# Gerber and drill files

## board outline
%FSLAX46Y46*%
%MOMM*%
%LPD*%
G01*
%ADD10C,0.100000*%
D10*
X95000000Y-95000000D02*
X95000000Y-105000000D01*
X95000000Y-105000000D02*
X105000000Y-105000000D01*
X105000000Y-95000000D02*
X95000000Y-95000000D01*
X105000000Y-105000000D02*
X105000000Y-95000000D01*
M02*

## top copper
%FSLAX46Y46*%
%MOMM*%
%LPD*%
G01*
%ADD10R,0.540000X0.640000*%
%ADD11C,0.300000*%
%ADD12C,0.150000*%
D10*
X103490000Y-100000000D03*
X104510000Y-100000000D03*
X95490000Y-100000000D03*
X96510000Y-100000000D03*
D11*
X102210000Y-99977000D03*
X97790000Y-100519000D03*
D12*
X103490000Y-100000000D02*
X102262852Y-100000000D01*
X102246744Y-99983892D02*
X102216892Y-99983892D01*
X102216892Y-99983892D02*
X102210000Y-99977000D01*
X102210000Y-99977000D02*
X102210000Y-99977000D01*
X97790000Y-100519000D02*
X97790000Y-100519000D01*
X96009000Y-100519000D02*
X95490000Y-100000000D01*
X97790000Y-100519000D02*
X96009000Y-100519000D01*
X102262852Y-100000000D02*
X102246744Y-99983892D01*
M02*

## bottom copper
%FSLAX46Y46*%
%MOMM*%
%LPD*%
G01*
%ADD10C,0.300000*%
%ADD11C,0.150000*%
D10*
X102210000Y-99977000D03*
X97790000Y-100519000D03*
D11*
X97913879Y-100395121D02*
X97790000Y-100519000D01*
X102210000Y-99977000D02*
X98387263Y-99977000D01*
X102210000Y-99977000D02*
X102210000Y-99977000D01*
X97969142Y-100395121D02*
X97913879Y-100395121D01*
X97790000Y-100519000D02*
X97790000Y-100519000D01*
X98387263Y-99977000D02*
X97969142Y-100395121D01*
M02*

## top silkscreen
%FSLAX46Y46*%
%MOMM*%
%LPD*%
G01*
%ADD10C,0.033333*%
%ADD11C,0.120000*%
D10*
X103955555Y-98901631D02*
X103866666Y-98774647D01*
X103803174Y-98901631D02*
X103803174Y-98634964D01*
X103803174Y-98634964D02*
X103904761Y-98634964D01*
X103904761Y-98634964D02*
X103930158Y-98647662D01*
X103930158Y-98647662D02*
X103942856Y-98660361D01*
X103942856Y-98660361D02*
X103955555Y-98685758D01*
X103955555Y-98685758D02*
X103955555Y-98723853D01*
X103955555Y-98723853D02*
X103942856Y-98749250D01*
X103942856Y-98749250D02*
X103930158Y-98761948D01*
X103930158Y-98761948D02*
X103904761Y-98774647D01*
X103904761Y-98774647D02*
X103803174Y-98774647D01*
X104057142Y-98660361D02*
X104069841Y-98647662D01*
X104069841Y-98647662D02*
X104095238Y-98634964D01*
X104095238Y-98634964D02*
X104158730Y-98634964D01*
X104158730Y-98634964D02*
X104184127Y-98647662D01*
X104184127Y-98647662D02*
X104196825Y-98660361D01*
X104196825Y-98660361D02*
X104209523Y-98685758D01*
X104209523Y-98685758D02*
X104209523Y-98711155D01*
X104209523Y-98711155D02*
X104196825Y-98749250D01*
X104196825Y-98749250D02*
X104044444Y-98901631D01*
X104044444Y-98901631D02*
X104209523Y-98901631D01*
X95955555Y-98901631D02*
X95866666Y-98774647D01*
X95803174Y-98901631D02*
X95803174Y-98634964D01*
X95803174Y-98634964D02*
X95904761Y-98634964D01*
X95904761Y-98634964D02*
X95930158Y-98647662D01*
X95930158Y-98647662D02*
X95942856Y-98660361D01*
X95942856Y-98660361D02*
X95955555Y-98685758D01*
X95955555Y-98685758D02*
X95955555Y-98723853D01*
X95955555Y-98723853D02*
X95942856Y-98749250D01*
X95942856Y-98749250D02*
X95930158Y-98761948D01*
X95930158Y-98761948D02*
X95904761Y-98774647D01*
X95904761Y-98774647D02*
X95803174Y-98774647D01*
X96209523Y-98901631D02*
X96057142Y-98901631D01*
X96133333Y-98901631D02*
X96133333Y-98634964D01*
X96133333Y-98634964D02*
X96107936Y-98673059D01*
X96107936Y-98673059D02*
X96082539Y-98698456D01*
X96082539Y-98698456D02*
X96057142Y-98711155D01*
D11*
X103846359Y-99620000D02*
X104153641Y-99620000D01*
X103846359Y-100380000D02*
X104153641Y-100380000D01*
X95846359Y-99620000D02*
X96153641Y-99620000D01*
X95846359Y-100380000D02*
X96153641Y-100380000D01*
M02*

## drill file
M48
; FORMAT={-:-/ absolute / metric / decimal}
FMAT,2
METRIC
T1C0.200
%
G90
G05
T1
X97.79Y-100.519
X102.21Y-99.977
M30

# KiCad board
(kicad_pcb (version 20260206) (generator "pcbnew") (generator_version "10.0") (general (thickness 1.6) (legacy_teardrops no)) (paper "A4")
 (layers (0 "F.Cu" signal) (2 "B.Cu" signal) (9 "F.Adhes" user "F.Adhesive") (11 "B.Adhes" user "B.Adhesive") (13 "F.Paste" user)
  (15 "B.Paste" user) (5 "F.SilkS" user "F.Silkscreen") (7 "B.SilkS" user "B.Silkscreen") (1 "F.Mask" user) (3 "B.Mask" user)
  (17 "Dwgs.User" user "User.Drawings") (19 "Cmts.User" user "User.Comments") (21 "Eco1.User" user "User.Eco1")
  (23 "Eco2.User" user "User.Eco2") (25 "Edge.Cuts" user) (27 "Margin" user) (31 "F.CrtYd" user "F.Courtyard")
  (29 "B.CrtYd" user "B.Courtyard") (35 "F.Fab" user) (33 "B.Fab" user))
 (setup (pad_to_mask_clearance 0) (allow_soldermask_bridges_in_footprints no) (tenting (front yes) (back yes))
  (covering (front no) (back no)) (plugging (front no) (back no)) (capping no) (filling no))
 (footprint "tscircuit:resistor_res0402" (layer "F.Cu") (at 104 100)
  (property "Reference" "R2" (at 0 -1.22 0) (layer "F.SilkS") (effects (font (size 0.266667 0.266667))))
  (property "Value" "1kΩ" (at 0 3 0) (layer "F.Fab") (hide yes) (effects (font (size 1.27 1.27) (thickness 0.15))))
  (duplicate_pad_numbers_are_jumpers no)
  (fp_line (start -0.153641 -0.38) (end 0.153641 -0.38) (stroke (width 0.12) (type default)) (layer "F.SilkS"))
  (fp_line (start -0.153641 0.38) (end 0.153641 0.38) (stroke (width 0.12) (type default)) (layer "F.SilkS"))
  (pad "1" smd rect (at -0.51 0) (size 0.54 0.64) (layers "F.Cu" "F.Mask" "F.Paste") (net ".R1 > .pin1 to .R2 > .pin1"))
  (pad "2" smd rect (at 0.51 0) (size 0.54 0.64) (layers "F.Cu" "F.Mask" "F.Paste")))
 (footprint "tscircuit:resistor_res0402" (layer "F.Cu") (at 96 100)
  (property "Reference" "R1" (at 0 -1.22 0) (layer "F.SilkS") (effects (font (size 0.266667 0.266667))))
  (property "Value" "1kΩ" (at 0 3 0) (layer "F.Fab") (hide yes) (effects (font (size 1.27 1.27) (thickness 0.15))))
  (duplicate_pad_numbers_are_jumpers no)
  (fp_line (start -0.153641 -0.38) (end 0.153641 -0.38) (stroke (width 0.12) (type default)) (layer "F.SilkS"))
  (fp_line (start -0.153641 0.38) (end 0.153641 0.38) (stroke (width 0.12) (type default)) (layer "F.SilkS"))
  (pad "1" smd rect (at -0.51 0) (size 0.54 0.64) (layers "F.Cu" "F.Mask" "F.Paste") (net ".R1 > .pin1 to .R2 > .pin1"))
  (pad "2" smd rect (at 0.51 0) (size 0.54 0.64) (layers "F.Cu" "F.Mask" "F.Paste")))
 (gr_line (start 95 95) (end 95 105) (stroke (width 0.1) (type solid)) (layer "Edge.Cuts"))
 (gr_line (start 95 105) (end 105 105) (stroke (width 0.1) (type solid)) (layer "Edge.Cuts"))
 (gr_line (start 105 95) (end 95 95) (stroke (width 0.1) (type solid)) (layer "Edge.Cuts"))
 (gr_line (start 105 105) (end 105 95) (stroke (width 0.1) (type solid)) (layer "Edge.Cuts"))
 (segment (start 103.49 100) (end 102.262852 100) (width 0.15) (layer "F.Cu") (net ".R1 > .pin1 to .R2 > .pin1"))
 (segment (start 102.246744 99.983892) (end 102.216892 99.983892) (width 0.15) (layer "F.Cu") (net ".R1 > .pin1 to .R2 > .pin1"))
 (segment (start 102.216892 99.983892) (end 102.21 99.977) (width 0.15) (layer "F.Cu") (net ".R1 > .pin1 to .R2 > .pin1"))
 (segment (start 102.21 99.977) (end 102.21 99.977) (width 0.15) (layer "F.Cu") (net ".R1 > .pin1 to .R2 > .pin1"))
 (segment (start 97.79 100.519) (end 97.79 100.519) (width 0.15) (layer "F.Cu") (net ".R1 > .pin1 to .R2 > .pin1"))
 (segment (start 96.009 100.519) (end 95.49 100) (width 0.15) (layer "F.Cu") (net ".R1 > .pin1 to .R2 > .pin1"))
 (segment (start 97.79 100.519) (end 96.009 100.519) (width 0.15) (layer "F.Cu") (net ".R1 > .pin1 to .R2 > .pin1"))
 (segment (start 102.262852 100) (end 102.246744 99.983892) (width 0.15) (layer "F.Cu") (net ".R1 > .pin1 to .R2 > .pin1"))
 (via (at 102.21 99.977) (size 0.3) (drill 0.2) (layers "F.Cu" "B.Cu") (capping no) (covering (front no) (back no))
  (plugging (front no) (back no)) (filling no) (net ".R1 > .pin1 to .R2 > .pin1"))
 (via (at 97.79 100.519) (size 0.3) (drill 0.2) (layers "F.Cu" "B.Cu") (capping no) (covering (front no) (back no))
  (plugging (front no) (back no)) (filling no) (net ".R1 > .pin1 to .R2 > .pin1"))
 (segment (start 97.913879 100.395121) (end 97.79 100.519) (width 0.15) (layer "B.Cu") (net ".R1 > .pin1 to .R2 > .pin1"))
 (segment (start 102.21 99.977) (end 98.387263 99.977) (width 0.15) (layer "B.Cu") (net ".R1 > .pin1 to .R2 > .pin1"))
 (segment (start 102.21 99.977) (end 102.21 99.977) (width 0.15) (layer "B.Cu") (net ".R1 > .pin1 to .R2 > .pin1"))
 (segment (start 97.969142 100.395121) (end 97.913879 100.395121) (width 0.15) (layer "B.Cu") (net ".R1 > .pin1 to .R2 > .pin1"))
 (segment (start 97.79 100.519) (end 97.79 100.519) (width 0.15) (layer "B.Cu") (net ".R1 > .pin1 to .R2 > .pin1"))
 (segment (start 98.387263 99.977) (end 97.969142 100.395121) (width 0.15) (layer "B.Cu") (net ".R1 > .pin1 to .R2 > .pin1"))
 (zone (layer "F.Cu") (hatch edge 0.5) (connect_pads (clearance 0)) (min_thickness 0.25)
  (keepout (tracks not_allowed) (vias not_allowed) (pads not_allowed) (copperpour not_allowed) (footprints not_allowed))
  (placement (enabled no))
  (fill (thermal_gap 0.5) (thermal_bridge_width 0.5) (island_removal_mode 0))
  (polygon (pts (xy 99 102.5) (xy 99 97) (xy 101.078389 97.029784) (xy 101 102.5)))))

